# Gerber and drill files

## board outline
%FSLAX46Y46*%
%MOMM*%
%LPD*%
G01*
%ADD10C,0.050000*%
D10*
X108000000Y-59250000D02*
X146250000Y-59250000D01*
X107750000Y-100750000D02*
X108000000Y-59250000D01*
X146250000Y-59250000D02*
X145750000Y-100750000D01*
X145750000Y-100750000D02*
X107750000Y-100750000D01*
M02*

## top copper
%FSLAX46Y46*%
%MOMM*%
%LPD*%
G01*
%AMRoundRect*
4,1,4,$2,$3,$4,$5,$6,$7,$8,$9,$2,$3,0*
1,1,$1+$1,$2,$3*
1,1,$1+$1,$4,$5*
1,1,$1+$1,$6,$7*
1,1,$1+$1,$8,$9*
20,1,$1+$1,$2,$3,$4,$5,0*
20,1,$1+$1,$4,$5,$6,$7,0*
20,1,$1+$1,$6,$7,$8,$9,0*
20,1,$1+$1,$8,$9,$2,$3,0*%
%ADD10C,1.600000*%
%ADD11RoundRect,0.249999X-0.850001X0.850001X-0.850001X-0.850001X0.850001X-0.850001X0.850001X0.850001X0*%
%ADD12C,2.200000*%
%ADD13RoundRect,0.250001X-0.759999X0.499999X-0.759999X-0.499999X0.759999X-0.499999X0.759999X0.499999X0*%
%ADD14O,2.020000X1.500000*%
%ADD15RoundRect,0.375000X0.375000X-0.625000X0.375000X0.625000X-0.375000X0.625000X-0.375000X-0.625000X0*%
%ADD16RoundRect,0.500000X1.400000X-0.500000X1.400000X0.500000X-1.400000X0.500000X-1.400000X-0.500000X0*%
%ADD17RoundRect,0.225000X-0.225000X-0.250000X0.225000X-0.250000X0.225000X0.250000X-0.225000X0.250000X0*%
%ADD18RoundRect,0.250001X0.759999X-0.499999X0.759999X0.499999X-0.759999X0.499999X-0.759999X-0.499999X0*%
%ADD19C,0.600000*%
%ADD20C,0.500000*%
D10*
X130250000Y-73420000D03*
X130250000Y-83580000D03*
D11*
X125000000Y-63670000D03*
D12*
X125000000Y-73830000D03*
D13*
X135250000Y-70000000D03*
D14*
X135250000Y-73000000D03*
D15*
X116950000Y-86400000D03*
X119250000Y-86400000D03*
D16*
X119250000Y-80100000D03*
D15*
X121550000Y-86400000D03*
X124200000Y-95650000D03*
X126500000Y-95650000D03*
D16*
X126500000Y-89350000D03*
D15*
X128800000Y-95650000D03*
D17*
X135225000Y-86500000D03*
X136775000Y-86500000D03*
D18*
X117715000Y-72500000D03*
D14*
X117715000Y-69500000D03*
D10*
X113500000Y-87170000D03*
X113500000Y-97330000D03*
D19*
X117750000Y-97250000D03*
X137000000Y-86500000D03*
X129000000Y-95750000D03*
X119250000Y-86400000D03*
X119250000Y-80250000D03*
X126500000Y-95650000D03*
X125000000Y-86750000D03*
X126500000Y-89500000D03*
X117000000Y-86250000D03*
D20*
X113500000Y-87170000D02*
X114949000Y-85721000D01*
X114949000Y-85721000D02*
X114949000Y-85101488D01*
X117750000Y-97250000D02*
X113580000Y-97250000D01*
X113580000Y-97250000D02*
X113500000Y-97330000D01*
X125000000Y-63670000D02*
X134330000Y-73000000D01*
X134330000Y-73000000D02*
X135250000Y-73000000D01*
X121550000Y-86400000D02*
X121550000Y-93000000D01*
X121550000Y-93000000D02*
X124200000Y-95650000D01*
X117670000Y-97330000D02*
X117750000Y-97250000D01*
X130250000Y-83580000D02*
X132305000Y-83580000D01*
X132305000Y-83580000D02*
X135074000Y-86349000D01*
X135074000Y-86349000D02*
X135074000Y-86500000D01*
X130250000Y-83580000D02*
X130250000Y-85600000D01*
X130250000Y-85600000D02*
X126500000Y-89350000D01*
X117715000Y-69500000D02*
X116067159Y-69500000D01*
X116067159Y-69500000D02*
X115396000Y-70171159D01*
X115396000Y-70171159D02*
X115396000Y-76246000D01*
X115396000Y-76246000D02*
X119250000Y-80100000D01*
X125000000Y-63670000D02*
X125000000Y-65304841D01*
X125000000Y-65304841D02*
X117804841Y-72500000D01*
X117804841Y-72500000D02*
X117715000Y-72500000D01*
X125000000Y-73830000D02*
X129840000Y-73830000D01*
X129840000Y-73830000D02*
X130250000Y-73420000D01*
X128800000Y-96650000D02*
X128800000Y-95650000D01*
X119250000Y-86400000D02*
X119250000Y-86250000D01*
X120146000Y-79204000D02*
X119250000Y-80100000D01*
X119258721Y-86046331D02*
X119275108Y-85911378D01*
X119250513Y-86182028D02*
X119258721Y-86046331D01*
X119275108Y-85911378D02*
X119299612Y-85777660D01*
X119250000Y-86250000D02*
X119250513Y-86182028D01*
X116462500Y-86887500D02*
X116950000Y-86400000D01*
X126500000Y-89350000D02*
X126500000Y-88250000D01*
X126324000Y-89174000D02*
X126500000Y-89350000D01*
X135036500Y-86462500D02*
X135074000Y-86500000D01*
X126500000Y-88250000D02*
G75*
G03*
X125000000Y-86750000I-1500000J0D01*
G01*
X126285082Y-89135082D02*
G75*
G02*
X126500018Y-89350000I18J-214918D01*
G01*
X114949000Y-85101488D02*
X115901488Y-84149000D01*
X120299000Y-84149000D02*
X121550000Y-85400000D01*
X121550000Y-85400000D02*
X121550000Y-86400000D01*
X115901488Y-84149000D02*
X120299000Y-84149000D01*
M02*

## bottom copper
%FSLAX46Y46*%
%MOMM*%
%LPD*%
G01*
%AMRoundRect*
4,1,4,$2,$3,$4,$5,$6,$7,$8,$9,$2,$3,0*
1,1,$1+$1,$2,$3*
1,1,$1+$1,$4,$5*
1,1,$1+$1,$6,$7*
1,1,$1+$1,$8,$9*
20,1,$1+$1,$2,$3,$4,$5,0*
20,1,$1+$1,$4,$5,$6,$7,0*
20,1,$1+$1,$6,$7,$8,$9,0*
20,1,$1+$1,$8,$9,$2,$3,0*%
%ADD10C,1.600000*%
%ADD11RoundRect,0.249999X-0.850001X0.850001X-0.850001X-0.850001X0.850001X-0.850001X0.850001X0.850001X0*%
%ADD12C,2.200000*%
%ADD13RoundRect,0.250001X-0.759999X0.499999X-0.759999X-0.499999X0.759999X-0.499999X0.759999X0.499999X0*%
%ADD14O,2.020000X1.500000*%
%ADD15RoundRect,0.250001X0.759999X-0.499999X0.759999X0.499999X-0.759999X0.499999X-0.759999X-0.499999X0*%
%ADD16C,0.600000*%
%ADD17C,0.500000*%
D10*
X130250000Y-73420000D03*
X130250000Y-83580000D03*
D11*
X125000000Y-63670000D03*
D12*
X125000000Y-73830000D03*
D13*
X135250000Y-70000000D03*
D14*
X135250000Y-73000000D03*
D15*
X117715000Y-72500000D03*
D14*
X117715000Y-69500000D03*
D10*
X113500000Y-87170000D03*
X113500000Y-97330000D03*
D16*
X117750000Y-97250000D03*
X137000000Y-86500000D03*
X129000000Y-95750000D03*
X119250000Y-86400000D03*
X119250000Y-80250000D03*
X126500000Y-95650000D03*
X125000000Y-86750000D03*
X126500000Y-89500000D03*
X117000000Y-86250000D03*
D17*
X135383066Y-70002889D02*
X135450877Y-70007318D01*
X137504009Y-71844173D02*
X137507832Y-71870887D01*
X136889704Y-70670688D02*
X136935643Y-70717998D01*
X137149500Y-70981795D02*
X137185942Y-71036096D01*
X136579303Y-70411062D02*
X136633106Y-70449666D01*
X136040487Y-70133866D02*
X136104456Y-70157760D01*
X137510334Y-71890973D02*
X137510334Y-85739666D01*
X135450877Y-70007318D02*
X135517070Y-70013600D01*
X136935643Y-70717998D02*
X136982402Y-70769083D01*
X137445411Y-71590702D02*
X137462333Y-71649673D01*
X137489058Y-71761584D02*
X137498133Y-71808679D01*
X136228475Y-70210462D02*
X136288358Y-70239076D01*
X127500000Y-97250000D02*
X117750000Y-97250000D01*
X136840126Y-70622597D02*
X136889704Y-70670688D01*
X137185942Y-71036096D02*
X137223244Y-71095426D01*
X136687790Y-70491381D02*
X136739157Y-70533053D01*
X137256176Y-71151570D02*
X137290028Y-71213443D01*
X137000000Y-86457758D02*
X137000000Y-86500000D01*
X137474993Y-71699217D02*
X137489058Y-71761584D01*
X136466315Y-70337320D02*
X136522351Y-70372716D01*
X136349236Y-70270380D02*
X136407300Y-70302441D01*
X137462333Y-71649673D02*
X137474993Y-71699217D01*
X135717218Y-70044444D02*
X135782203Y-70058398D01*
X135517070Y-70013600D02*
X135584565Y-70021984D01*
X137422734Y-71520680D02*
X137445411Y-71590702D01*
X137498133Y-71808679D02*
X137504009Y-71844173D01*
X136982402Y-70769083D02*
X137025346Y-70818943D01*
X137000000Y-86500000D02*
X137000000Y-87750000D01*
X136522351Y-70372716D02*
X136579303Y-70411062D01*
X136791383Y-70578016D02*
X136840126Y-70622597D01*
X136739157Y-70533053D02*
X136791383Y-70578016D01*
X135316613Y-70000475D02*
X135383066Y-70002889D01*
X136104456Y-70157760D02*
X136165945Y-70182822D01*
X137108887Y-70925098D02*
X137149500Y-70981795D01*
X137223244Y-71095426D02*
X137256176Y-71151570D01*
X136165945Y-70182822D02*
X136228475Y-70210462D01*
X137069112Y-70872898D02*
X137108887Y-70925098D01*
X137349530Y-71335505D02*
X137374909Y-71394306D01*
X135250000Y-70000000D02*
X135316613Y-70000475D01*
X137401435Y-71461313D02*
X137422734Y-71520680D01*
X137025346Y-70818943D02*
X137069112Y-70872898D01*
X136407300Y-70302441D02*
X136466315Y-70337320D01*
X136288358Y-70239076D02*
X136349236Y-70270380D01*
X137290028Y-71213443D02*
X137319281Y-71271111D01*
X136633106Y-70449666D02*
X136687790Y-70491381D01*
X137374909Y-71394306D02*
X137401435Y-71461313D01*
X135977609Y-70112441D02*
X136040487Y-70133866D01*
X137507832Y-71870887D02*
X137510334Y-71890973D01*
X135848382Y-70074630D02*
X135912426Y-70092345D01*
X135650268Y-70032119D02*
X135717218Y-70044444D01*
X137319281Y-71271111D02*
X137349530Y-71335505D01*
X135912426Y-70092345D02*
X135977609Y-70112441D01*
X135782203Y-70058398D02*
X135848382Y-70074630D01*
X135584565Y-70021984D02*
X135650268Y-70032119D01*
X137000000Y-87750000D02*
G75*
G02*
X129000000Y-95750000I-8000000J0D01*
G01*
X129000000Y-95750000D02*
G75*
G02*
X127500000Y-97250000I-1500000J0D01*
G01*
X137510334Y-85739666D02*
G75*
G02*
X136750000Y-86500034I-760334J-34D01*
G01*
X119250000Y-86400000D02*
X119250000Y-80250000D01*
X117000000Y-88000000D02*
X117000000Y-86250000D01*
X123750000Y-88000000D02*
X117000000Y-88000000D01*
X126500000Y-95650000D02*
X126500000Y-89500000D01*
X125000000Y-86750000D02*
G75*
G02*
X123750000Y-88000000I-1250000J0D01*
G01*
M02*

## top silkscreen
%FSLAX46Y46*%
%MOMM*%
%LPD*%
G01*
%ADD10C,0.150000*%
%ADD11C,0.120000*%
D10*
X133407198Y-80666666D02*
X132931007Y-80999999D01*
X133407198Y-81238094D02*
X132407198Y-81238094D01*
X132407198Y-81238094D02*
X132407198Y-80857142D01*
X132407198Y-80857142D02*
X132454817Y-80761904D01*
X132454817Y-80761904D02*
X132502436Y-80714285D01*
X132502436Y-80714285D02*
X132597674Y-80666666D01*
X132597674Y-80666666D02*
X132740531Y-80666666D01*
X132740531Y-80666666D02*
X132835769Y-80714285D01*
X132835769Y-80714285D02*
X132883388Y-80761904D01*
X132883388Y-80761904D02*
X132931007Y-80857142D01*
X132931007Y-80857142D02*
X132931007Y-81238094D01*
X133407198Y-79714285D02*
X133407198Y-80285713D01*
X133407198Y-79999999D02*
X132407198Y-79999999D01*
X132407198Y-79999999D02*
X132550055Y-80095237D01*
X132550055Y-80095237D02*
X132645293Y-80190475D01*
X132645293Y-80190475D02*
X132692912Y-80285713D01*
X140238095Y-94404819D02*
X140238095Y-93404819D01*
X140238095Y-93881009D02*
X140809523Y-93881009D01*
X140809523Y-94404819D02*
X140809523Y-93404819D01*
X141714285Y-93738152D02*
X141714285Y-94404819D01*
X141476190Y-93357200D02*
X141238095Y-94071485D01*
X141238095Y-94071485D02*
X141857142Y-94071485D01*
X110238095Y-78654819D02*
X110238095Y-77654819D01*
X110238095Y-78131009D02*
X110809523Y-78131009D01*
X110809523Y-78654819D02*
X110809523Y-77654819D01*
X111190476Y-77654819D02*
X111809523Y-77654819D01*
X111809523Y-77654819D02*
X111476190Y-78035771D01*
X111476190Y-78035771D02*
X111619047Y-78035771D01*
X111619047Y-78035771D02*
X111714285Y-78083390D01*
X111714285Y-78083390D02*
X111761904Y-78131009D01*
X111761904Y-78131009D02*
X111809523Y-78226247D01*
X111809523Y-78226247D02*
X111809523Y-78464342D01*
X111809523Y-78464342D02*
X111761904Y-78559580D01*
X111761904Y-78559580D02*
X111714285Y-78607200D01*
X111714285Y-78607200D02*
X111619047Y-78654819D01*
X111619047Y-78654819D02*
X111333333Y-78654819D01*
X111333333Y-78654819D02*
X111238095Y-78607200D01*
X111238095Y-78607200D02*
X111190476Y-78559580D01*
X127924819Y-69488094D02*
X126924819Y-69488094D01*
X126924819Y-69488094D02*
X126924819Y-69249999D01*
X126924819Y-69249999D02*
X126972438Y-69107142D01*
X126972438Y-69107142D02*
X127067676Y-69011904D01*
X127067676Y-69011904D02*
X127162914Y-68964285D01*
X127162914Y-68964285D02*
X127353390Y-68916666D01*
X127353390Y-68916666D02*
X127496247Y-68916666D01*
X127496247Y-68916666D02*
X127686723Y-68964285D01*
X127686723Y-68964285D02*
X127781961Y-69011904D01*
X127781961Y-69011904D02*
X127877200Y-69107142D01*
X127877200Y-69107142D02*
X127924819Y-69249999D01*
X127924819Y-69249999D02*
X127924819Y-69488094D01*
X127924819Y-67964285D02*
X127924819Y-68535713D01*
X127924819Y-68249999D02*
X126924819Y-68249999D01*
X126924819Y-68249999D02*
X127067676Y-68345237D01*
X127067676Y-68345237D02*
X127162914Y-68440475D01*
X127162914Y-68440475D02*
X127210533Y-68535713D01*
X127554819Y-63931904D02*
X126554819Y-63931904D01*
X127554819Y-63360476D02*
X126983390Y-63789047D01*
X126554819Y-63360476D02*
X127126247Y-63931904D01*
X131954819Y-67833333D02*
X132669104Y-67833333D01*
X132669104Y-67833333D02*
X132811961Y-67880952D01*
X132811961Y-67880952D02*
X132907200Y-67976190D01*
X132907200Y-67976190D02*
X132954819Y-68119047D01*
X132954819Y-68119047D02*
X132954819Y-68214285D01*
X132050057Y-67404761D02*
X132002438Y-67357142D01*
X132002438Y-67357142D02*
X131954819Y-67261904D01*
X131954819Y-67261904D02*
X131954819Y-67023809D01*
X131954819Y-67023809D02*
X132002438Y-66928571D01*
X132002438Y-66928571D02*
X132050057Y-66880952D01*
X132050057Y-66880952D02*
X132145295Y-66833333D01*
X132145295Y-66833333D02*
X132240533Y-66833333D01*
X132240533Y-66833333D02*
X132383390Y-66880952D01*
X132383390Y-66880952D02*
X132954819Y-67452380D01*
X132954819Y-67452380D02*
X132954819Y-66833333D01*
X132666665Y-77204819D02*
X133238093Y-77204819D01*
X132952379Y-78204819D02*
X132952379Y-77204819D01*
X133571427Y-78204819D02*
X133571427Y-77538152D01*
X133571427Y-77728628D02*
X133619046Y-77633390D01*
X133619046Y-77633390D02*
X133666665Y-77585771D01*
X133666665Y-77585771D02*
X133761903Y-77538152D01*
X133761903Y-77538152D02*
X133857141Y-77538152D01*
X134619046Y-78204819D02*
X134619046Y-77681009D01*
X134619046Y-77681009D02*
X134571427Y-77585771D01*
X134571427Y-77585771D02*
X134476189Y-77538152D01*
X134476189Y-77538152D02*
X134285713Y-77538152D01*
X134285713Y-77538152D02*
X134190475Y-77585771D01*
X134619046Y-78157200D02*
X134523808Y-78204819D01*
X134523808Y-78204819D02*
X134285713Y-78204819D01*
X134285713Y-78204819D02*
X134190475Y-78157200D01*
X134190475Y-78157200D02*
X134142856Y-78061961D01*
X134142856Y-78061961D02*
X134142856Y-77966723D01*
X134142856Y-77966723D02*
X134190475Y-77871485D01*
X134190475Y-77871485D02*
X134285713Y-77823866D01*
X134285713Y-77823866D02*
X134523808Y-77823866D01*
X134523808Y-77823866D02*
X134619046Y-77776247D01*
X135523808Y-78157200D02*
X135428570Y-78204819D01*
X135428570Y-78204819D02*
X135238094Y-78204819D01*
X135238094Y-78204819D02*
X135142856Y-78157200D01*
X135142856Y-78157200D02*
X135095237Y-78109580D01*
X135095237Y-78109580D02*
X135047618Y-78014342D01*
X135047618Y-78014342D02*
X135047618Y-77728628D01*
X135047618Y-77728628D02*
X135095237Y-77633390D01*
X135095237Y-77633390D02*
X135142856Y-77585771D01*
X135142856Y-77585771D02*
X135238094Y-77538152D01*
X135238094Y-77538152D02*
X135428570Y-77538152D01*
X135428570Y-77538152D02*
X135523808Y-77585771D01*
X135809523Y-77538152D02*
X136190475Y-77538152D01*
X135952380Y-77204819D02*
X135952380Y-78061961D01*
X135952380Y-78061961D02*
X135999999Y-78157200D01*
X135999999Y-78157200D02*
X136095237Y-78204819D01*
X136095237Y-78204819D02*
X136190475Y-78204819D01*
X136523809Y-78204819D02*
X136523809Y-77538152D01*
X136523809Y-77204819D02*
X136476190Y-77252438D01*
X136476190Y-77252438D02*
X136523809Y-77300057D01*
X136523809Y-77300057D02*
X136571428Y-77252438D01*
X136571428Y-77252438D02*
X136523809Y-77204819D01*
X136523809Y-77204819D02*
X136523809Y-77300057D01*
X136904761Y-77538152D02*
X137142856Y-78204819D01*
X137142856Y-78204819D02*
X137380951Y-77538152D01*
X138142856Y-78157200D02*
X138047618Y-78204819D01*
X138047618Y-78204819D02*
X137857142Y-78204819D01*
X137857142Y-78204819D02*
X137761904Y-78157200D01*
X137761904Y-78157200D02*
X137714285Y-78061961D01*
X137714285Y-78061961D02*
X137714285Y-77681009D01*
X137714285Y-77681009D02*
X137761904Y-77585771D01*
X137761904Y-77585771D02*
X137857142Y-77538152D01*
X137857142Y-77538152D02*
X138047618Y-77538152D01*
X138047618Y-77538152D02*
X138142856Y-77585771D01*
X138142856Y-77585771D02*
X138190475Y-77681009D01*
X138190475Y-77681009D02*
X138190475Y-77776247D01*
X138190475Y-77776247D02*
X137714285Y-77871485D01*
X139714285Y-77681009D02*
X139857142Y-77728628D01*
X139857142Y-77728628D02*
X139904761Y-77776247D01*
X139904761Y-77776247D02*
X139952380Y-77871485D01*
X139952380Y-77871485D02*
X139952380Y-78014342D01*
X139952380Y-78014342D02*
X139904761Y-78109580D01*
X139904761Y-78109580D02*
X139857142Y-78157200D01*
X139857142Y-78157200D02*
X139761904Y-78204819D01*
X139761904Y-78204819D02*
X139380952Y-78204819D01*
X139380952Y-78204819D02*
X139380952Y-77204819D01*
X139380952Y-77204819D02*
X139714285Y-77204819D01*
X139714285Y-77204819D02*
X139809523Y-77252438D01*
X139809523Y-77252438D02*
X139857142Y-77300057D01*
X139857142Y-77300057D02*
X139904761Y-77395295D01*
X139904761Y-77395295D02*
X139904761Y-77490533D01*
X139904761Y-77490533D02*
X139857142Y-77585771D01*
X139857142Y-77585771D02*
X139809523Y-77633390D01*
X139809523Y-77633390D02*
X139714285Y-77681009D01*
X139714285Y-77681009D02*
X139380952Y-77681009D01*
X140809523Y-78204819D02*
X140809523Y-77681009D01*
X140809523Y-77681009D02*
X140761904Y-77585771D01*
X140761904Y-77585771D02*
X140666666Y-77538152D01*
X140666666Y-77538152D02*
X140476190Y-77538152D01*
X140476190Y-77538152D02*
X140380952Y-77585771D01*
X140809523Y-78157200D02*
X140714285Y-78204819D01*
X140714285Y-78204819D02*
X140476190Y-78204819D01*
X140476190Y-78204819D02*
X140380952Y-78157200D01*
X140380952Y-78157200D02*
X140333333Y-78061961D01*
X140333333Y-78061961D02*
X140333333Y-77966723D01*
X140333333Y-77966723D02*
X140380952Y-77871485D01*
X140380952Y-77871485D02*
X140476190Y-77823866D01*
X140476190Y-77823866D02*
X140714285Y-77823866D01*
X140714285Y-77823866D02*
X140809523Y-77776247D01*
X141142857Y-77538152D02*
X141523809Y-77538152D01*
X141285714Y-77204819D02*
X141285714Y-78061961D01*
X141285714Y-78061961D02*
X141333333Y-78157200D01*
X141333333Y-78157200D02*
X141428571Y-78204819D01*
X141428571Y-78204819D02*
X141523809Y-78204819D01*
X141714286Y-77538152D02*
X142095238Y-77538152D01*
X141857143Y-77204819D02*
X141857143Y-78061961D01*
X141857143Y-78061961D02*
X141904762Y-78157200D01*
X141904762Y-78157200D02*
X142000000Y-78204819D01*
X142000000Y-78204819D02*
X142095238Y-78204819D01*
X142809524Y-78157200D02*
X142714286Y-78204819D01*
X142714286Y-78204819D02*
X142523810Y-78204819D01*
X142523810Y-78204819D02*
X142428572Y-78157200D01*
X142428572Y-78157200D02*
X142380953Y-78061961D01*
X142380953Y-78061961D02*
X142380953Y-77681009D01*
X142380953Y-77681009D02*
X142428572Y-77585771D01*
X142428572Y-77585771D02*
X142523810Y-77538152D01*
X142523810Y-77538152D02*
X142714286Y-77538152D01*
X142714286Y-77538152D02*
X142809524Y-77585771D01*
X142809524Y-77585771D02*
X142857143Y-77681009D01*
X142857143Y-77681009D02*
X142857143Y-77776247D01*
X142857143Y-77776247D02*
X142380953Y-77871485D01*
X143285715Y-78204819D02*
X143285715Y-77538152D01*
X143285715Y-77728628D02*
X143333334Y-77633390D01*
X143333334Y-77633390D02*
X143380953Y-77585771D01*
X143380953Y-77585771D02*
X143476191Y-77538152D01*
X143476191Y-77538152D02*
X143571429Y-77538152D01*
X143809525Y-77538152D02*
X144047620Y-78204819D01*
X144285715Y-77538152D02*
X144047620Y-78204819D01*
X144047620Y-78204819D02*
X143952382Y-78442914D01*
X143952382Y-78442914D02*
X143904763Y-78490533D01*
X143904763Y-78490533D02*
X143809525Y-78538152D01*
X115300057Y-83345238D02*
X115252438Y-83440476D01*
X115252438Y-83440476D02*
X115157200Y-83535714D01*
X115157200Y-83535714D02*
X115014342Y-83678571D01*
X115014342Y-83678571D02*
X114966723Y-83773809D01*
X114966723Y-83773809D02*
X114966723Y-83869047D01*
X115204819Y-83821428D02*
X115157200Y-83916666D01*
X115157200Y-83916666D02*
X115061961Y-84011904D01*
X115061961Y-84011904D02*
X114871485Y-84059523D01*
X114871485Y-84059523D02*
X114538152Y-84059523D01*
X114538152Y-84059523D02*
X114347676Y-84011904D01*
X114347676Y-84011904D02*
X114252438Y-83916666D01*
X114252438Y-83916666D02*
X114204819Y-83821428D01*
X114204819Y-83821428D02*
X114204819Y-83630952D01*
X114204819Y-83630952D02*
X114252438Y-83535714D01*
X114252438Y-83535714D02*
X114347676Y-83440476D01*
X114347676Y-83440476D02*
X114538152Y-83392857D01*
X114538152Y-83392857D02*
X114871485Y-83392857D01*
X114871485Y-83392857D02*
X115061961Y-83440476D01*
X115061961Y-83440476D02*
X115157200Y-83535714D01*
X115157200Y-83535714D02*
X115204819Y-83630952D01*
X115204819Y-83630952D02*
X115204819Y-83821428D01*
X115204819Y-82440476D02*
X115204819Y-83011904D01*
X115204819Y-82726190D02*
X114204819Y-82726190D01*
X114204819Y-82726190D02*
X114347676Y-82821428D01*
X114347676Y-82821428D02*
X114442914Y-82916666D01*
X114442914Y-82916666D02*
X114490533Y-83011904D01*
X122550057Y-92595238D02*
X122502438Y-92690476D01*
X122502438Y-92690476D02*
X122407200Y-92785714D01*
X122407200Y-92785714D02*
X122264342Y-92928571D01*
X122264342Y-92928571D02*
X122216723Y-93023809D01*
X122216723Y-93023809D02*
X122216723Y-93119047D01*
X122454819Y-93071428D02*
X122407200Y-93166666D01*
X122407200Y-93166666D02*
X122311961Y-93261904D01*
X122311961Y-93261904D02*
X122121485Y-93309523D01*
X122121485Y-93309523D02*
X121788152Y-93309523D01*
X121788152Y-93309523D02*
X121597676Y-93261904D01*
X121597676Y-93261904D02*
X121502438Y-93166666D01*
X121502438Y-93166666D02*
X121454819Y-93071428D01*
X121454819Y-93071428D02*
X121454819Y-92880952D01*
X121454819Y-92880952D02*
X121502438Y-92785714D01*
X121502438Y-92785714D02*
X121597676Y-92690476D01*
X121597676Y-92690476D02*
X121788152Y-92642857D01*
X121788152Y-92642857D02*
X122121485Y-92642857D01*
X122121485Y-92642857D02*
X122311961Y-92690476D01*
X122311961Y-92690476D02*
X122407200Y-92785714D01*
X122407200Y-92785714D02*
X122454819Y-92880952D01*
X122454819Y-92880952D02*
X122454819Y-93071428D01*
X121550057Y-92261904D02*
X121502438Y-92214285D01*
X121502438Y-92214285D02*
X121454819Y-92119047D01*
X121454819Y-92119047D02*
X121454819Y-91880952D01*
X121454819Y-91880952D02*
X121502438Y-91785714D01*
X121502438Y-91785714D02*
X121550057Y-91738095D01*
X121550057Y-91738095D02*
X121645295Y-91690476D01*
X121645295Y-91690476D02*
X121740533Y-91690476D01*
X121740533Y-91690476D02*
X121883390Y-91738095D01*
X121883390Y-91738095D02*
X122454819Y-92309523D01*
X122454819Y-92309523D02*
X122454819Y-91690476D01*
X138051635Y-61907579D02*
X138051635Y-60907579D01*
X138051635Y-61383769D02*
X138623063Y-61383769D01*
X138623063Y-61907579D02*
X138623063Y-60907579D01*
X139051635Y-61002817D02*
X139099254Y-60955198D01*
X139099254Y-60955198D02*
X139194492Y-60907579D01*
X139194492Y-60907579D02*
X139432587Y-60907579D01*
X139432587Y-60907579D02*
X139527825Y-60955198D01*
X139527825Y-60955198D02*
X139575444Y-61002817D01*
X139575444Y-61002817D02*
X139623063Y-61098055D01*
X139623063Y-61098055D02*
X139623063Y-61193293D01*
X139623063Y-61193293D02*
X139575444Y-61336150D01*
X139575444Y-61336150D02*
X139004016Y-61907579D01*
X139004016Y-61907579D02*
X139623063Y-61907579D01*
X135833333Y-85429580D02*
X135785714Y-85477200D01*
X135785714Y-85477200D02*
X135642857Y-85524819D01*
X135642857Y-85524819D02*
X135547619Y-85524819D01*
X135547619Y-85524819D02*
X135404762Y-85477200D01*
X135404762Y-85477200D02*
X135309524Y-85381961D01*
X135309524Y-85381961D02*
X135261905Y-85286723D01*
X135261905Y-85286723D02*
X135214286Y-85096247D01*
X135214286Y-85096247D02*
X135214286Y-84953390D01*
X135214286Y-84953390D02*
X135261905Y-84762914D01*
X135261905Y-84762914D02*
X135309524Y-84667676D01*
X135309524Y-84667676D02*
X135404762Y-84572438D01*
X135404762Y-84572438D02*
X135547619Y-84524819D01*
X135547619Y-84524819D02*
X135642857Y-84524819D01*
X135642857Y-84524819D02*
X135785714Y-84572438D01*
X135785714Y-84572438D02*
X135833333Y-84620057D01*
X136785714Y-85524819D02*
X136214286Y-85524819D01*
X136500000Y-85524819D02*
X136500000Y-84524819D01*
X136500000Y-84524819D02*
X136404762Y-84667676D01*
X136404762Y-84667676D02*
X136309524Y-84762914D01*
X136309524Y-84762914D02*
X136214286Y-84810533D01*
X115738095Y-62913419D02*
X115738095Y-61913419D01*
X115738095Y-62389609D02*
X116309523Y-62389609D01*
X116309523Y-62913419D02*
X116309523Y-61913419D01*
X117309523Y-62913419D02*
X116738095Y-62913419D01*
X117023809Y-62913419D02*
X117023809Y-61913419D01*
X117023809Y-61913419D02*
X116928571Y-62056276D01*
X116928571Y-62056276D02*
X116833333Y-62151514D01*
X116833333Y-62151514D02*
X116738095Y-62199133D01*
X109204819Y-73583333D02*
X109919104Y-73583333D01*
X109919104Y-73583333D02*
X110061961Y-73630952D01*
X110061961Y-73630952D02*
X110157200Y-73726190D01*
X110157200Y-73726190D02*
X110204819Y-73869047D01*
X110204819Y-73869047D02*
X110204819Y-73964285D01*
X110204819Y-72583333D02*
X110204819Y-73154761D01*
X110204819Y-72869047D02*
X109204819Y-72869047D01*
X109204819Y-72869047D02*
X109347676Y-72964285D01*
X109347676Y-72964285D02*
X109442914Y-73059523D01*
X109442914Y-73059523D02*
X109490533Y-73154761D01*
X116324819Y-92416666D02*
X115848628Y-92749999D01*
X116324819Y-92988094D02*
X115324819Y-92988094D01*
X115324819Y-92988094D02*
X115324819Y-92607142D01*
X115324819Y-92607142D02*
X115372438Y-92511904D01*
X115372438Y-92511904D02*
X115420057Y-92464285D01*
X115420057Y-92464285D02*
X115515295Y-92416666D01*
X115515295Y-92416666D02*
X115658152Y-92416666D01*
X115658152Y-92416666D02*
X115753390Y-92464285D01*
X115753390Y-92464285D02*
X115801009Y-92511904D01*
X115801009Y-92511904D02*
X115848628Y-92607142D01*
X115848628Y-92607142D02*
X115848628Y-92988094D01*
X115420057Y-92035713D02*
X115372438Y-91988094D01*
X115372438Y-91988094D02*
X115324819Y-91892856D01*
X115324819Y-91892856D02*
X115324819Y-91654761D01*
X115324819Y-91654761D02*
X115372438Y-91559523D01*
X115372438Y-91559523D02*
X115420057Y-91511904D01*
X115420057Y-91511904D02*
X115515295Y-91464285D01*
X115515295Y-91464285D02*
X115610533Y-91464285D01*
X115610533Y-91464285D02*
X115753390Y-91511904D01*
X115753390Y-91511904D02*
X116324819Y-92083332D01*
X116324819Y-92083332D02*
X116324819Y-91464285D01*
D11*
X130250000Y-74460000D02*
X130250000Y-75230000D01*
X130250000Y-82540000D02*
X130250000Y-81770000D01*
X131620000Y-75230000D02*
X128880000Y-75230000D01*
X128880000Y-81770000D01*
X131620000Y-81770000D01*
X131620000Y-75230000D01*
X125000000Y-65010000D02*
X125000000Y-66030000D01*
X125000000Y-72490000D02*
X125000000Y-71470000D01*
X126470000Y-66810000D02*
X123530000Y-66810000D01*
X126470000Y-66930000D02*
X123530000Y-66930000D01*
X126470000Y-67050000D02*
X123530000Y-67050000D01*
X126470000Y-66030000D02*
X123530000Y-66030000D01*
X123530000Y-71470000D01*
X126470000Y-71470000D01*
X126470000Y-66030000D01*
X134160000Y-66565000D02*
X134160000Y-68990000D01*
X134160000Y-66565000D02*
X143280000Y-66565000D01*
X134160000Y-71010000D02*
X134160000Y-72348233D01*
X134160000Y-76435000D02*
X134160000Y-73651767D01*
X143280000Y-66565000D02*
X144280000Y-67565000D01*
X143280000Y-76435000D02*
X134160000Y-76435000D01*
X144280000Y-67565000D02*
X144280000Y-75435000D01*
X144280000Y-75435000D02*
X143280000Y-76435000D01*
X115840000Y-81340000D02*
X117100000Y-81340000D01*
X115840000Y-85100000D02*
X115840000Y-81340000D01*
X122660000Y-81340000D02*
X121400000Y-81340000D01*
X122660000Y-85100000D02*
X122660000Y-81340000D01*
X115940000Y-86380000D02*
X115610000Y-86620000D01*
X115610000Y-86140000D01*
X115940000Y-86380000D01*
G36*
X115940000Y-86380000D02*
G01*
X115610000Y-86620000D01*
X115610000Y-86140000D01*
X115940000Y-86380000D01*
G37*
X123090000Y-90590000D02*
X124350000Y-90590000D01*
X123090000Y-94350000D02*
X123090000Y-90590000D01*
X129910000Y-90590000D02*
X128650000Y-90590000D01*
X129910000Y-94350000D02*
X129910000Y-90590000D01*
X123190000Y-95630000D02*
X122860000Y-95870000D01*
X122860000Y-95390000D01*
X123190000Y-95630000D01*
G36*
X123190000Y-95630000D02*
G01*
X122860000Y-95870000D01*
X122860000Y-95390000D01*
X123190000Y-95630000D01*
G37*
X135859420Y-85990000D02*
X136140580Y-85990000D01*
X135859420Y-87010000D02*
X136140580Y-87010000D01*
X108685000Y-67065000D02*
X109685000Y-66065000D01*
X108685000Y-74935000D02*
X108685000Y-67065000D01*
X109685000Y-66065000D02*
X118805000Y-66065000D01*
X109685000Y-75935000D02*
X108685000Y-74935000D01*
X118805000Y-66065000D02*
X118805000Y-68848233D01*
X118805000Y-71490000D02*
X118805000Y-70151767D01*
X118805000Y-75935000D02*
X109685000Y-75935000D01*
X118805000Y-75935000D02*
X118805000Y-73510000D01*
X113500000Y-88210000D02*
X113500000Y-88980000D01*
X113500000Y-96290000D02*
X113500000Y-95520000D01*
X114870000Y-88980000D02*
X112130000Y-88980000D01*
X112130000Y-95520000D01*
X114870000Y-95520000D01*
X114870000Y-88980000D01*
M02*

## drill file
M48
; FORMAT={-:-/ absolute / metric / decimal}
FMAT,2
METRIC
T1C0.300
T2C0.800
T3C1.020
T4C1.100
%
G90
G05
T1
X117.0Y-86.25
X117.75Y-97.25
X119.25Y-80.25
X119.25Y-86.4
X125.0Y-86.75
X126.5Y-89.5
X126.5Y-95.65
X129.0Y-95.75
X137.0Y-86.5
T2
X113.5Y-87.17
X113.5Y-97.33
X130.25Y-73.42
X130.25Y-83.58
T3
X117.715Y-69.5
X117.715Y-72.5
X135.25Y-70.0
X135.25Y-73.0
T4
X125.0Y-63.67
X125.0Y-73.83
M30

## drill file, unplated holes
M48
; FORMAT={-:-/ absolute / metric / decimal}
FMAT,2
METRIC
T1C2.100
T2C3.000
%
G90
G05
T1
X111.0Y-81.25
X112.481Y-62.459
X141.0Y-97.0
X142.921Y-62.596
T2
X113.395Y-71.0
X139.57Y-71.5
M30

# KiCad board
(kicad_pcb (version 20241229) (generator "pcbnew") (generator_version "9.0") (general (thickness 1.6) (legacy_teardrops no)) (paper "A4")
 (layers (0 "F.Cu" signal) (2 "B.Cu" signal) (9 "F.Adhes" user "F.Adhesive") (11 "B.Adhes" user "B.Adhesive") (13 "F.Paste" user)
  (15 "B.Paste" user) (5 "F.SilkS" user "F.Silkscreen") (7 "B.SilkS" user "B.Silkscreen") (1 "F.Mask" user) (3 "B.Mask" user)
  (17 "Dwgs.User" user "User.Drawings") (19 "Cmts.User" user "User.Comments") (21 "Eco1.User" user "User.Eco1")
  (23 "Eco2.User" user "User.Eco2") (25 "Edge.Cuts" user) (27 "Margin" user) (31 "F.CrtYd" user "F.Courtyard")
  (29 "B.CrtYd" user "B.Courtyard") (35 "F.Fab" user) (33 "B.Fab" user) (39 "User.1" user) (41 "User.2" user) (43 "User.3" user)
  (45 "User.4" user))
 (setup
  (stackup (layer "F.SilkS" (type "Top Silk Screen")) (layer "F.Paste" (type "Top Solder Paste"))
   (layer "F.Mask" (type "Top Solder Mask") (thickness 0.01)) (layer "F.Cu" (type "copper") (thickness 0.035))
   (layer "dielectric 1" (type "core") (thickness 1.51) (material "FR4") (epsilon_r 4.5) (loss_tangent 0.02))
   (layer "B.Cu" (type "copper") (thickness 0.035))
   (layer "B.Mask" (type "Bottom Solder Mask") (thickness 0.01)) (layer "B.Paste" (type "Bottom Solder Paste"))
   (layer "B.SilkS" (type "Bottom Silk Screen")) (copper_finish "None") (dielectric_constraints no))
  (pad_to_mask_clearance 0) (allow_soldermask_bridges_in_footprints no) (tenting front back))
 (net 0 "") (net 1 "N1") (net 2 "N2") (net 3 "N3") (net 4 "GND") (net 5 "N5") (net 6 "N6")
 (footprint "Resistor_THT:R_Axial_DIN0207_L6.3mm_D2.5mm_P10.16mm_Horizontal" (layer "F.Cu") (at 130.25 73.42 -90)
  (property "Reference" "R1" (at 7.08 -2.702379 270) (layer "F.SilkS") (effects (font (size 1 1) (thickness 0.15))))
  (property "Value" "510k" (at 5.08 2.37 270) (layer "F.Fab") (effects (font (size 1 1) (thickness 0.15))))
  (fp_line (start 1.04 0) (end 1.81 0) (stroke (width 0.12) (type solid)) (layer "F.SilkS"))
  (fp_line (start 9.12 0) (end 8.35 0) (stroke (width 0.12) (type solid)) (layer "F.SilkS"))
  (fp_rect (start 1.81 -1.37) (end 8.35 1.37) (stroke (width 0.12) (type solid)) (fill no) (layer "F.SilkS"))
  (pad "1" thru_hole circle (at 0 0 270) (size 1.6 1.6) (drill 0.8) (layers "*.Cu" "*.Mask") (remove_unused_layers no) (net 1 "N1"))
  (pad "2" thru_hole circle (at 10.16 0 270) (size 1.6 1.6) (drill 0.8) (layers "*.Cu" "*.Mask") (remove_unused_layers no) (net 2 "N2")))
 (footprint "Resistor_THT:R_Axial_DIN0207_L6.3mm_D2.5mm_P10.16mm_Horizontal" (layer "F.Cu") (at 113.5 87.17 -90)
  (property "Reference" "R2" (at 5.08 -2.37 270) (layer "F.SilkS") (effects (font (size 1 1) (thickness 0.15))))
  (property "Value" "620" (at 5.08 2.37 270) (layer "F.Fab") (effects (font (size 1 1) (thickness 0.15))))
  (fp_line (start 1.04 0) (end 1.81 0) (stroke (width 0.12) (type solid)) (layer "F.SilkS"))
  (fp_line (start 9.12 0) (end 8.35 0) (stroke (width 0.12) (type solid)) (layer "F.SilkS"))
  (fp_rect (start 1.81 -1.37) (end 8.35 1.37) (stroke (width 0.12) (type solid)) (fill no) (layer "F.SilkS"))
  (pad "1" thru_hole circle (at 0 0 270) (size 1.6 1.6) (drill 0.8) (layers "*.Cu" "*.Mask") (remove_unused_layers no) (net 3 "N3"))
  (pad "2" thru_hole circle (at 10.16 0 270) (size 1.6 1.6) (drill 0.8) (layers "*.Cu" "*.Mask") (remove_unused_layers no) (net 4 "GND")))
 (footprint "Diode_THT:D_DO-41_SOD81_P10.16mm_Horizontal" (layer "F.Cu") (at 125 63.67 -90)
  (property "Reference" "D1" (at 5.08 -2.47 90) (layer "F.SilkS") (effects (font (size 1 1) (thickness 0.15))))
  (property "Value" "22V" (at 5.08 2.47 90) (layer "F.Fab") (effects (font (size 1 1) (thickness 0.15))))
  (fp_line (start 1.34 0) (end 2.36 0) (stroke (width 0.12) (type solid)) (layer "F.SilkS"))
  (fp_line (start 8.82 0) (end 7.8 0) (stroke (width 0.12) (type solid)) (layer "F.SilkS"))
  (fp_line (start 3.14 -1.47) (end 3.14 1.47) (stroke (width 0.12) (type solid)) (layer "F.SilkS"))
  (fp_line (start 3.26 -1.47) (end 3.26 1.47) (stroke (width 0.12) (type solid)) (layer "F.SilkS"))
  (fp_line (start 3.38 -1.47) (end 3.38 1.47) (stroke (width 0.12) (type solid)) (layer "F.SilkS"))
  (fp_rect (start 2.36 -1.47) (end 7.8 1.47) (stroke (width 0.12) (type solid)) (fill no) (layer "F.SilkS"))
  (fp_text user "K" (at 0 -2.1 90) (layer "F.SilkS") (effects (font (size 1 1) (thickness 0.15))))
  (pad "1" thru_hole roundrect (at 0 0 270) (size 2.2 2.2) (drill 1.1) (layers "*.Cu" "*.Mask") (remove_unused_layers no)
   (roundrect_rratio 0.113636) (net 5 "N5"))
  (pad "2" thru_hole circle (at 10.16 0 270) (size 2.2 2.2) (drill 1.1) (layers "*.Cu" "*.Mask") (remove_unused_layers no) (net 1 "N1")))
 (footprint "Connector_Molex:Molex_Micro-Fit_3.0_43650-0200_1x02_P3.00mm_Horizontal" (layer "F.Cu") (at 135.25 70 -90)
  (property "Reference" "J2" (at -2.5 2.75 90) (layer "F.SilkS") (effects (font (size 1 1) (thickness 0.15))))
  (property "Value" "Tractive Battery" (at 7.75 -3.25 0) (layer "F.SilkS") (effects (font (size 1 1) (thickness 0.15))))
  (fp_line (start -3.435 1.09) (end -1.01 1.09) (stroke (width 0.12) (type solid)) (layer "F.SilkS"))
  (fp_line (start -3.435 1.09) (end -3.435 -8.03) (stroke (width 0.12) (type solid)) (layer "F.SilkS"))
  (fp_line (start 1.01 1.09) (end 2.348233 1.09) (stroke (width 0.12) (type solid)) (layer "F.SilkS"))
  (fp_line (start 6.435 1.09) (end 3.651767 1.09) (stroke (width 0.12) (type solid)) (layer "F.SilkS"))
  (fp_line (start -3.435 -8.03) (end -2.435 -9.03) (stroke (width 0.12) (type solid)) (layer "F.SilkS"))
  (fp_line (start 6.435 -8.03) (end 6.435 1.09) (stroke (width 0.12) (type solid)) (layer "F.SilkS"))
  (fp_line (start -2.435 -9.03) (end 5.435 -9.03) (stroke (width 0.12) (type solid)) (layer "F.SilkS"))
  (fp_line (start 5.435 -9.03) (end 6.435 -8.03) (stroke (width 0.12) (type solid)) (layer "F.SilkS"))
  (pad "" np_thru_hole circle (at 1.5 -4.32 270) (size 3 3) (drill 3) (layers "*.Cu" "*.Mask"))
  (pad "1" thru_hole roundrect (at 0 0 270) (size 1.5 2.02) (drill 1.02) (layers "*.Cu" "*.Mask") (remove_unused_layers no)
   (roundrect_rratio 0.166667) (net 4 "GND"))
  (pad "2" thru_hole oval (at 3 0 270) (size 1.5 2.02) (drill 1.02) (layers "*.Cu" "*.Mask") (remove_unused_layers no) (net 5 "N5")))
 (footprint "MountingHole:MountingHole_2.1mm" (layer "F.Cu") (at 111 81.25)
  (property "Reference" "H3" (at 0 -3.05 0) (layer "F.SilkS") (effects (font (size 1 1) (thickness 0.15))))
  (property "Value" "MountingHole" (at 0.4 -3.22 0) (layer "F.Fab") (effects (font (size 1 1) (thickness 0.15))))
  (pad "" np_thru_hole circle (at 0 0) (size 2.1 2.1) (drill 2.1) (layers "*.Cu" "*.Mask")))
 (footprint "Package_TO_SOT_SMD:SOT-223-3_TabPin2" (layer "F.Cu") (at 119.25 83.25 90)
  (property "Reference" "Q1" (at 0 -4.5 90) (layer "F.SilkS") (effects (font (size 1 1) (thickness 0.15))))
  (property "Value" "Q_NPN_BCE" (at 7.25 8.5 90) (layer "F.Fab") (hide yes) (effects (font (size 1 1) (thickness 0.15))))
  (fp_line (start 1.91 -3.41) (end 1.91 -2.15) (stroke (width 0.12) (type solid)) (layer "F.SilkS"))
  (fp_line (start -1.85 -3.41) (end 1.91 -3.41) (stroke (width 0.12) (type solid)) (layer "F.SilkS"))
  (fp_line (start 1.91 3.41) (end 1.91 2.15) (stroke (width 0.12) (type solid)) (layer "F.SilkS"))
  (fp_line (start -1.85 3.41) (end 1.91 3.41) (stroke (width 0.12) (type solid)) (layer "F.SilkS"))
  (fp_poly
   (pts (xy -3.13 -3.31) (xy -3.37 -3.64) (xy -2.89 -3.64) (xy -3.13 -3.31)) (stroke (width 0.12) (type solid)) (fill yes) (layer "F.SilkS"))
  (pad "1" smd roundrect (at -3.15 -2.3 90) (size 2 1.5) (layers "F.Cu" "F.Mask" "F.Paste") (roundrect_rratio 0.25) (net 2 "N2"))
  (pad "2" smd roundrect (at -3.15 0 90) (size 2 1.5) (layers "F.Cu" "F.Mask" "F.Paste") (roundrect_rratio 0.25) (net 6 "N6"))
  (pad "2" smd roundrect (at 3.15 0 90) (size 2 3.8) (layers "F.Cu" "F.Mask" "F.Paste") (roundrect_rratio 0.25) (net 6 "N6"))
  (pad "3" smd roundrect (at -3.15 2.3 90) (size 2 1.5) (layers "F.Cu" "F.Mask" "F.Paste") (roundrect_rratio 0.25) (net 3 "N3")))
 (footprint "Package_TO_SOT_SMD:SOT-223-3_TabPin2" (layer "F.Cu") (at 126.5 92.5 90)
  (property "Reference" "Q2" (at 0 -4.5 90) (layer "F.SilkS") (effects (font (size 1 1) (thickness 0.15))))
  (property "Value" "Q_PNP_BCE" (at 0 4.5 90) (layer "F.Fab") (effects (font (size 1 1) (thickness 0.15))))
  (fp_line (start 1.91 -3.41) (end 1.91 -2.15) (stroke (width 0.12) (type solid)) (layer "F.SilkS"))
  (fp_line (start -1.85 -3.41) (end 1.91 -3.41) (stroke (width 0.12) (type solid)) (layer "F.SilkS"))
  (fp_line (start 1.91 3.41) (end 1.91 2.15) (stroke (width 0.12) (type solid)) (layer "F.SilkS"))
  (fp_line (start -1.85 3.41) (end 1.91 3.41) (stroke (width 0.12) (type solid)) (layer "F.SilkS"))
  (fp_poly
   (pts (xy -3.13 -3.31) (xy -3.37 -3.64) (xy -2.89 -3.64) (xy -3.13 -3.31)) (stroke (width 0.12) (type solid)) (fill yes) (layer "F.SilkS"))
  (pad "1" smd roundrect (at -3.15 -2.3 90) (size 2 1.5) (layers "F.Cu" "F.Mask" "F.Paste") (roundrect_rratio 0.25) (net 3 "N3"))
  (pad "2" smd roundrect (at -3.15 0 90) (size 2 1.5) (layers "F.Cu" "F.Mask" "F.Paste") (roundrect_rratio 0.25) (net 2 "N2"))
  (pad "2" smd roundrect (at 3.15 0 90) (size 2 3.8) (layers "F.Cu" "F.Mask" "F.Paste") (roundrect_rratio 0.25) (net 2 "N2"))
  (pad "3" smd roundrect (at -3.15 2.3 90) (size 2 1.5) (layers "F.Cu" "F.Mask" "F.Paste") (roundrect_rratio 0.25) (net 4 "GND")))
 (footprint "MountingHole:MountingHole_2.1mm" (layer "F.Cu") (at 142.92072 62.59576)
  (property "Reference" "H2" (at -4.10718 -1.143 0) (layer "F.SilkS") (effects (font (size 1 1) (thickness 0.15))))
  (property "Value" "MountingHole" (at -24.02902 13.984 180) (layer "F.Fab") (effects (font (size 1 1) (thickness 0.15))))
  (pad "" np_thru_hole circle (at 0 0) (size 2.1 2.1) (drill 2.1) (layers "*.Cu" "*.Mask")))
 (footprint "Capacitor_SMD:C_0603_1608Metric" (layer "F.Cu") (at 136 86.5)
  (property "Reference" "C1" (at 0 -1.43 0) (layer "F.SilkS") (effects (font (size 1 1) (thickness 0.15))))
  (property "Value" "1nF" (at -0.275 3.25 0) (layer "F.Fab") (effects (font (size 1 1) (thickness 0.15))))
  (fp_line (start -0.14058 -0.51) (end 0.14058 -0.51) (stroke (width 0.12) (type solid)) (layer "F.SilkS"))
  (fp_line (start -0.14058 0.51) (end 0.14058 0.51) (stroke (width 0.12) (type solid)) (layer "F.SilkS"))
  (pad "1" smd roundrect (at -0.775 0) (size 0.9 0.95) (layers "F.Cu" "F.Mask" "F.Paste") (roundrect_rratio 0.25) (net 2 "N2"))
  (pad "2" smd roundrect (at 0.775 0) (size 0.9 0.95) (layers "F.Cu" "F.Mask" "F.Paste") (roundrect_rratio 0.25) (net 4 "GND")))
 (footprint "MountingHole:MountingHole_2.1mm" (layer "F.Cu") (at 112.48136 62.4586)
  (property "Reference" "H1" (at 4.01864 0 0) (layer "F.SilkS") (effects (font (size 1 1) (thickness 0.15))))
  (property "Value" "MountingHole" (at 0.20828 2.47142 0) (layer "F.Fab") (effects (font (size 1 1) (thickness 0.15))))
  (pad "" np_thru_hole circle (at 0 0) (size 2.1 2.1) (drill 2.1) (layers "*.Cu" "*.Mask")))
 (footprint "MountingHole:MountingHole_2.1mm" (layer "F.Cu") (at 141 97)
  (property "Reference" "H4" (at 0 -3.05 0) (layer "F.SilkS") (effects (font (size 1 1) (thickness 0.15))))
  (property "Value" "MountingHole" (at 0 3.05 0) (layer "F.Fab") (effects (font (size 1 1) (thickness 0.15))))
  (pad "" np_thru_hole circle (at 0 0) (size 2.1 2.1) (drill 2.1) (layers "*.Cu" "*.Mask")))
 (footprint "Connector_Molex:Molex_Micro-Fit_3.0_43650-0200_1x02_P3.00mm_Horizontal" (layer "F.Cu") (at 117.715 72.5 90)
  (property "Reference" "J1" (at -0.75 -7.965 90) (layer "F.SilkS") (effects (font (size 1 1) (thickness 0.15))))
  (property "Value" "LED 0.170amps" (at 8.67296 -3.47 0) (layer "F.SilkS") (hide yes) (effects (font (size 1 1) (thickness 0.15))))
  (fp_line (start 5.435 -9.03) (end 6.435 -8.03) (stroke (width 0.12) (type solid)) (layer "F.SilkS"))
  (fp_line (start -2.435 -9.03) (end 5.435 -9.03) (stroke (width 0.12) (type solid)) (layer "F.SilkS"))
  (fp_line (start 6.435 -8.03) (end 6.435 1.09) (stroke (width 0.12) (type solid)) (layer "F.SilkS"))
  (fp_line (start -3.435 -8.03) (end -2.435 -9.03) (stroke (width 0.12) (type solid)) (layer "F.SilkS"))
  (fp_line (start 6.435 1.09) (end 3.651767 1.09) (stroke (width 0.12) (type solid)) (layer "F.SilkS"))
  (fp_line (start 1.01 1.09) (end 2.348233 1.09) (stroke (width 0.12) (type solid)) (layer "F.SilkS"))
  (fp_line (start -3.435 1.09) (end -3.435 -8.03) (stroke (width 0.12) (type solid)) (layer "F.SilkS"))
  (fp_line (start -3.435 1.09) (end -1.01 1.09) (stroke (width 0.12) (type solid)) (layer "F.SilkS"))
  (pad "" np_thru_hole circle (at 1.5 -4.32 90) (size 3 3) (drill 3) (layers "*.Cu" "*.Mask"))
  (pad "1" thru_hole roundrect (at 0 0 90) (size 1.5 2.02) (drill 1.02) (layers "*.Cu" "*.Mask") (remove_unused_layers no)
   (roundrect_rratio 0.166667) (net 5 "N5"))
  (pad "2" thru_hole oval (at 3 0 90) (size 1.5 2.02) (drill 1.02) (layers "*.Cu" "*.Mask") (remove_unused_layers no) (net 6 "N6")))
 (gr_line (start 108 59.25) (end 146.25 59.25) (stroke (width 0.05) (type default)) (layer "Edge.Cuts"))
 (gr_line (start 107.75 100.75) (end 108 59.25) (stroke (width 0.05) (type default)) (layer "Edge.Cuts"))
 (gr_line (start 146.25 59.25) (end 145.75 100.75) (stroke (width 0.05) (type default)) (layer "Edge.Cuts"))
 (gr_line (start 145.75 100.75) (end 107.75 100.75) (stroke (width 0.05) (type default)) (layer "Edge.Cuts"))
 (segment (start 117.67 97.33) (end 117.75 97.25) (width 0.5) (layer "F.Cu") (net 4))
 (segment (start 113.58 97.25) (end 113.5 97.33) (width 0.5) (layer "F.Cu") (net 4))
 (segment (start 128.8 96.65) (end 128.8 95.65) (width 0.5) (layer "F.Cu") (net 4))
 (segment (start 117.75 97.25) (end 113.58 97.25) (width 0.5) (layer "F.Cu") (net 4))
 (via (at 117.75 97.25) (size 0.6) (drill 0.3) (layers "F.Cu" "B.Cu") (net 4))
 (via (at 137 86.5) (size 0.6) (drill 0.3) (layers "F.Cu" "B.Cu") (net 4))
 (via (at 129 95.75) (size 0.6) (drill 0.3) (layers "F.Cu" "B.Cu") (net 4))
 (segment (start 135.383066 70.002889) (end 135.450877 70.007318) (width 0.5) (layer "B.Cu") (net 4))
 (segment (start 137.504009 71.844173) (end 137.507832 71.870887) (width 0.5) (layer "B.Cu") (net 4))
 (segment (start 136.889704 70.670688) (end 136.935643 70.717998) (width 0.5) (layer "B.Cu") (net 4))
 (segment (start 137.1495 70.981795) (end 137.185942 71.036096) (width 0.5) (layer "B.Cu") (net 4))
 (segment (start 136.579303 70.411062) (end 136.633106 70.449666) (width 0.5) (layer "B.Cu") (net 4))
 (segment (start 136.040487 70.133866) (end 136.104456 70.15776) (width 0.5) (layer "B.Cu") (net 4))
 (segment (start 137.510334 71.890973) (end 137.510334 85.739666) (width 0.5) (layer "B.Cu") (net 4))
 (segment (start 135.450877 70.007318) (end 135.51707 70.0136) (width 0.5) (layer "B.Cu") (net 4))
 (segment (start 136.935643 70.717998) (end 136.982402 70.769083) (width 0.5) (layer "B.Cu") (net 4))
 (segment (start 137.445411 71.590702) (end 137.462333 71.649673) (width 0.5) (layer "B.Cu") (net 4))
 (segment (start 137.489058 71.761584) (end 137.498133 71.808679) (width 0.5) (layer "B.Cu") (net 4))
 (segment (start 136.228475 70.210462) (end 136.288358 70.239076) (width 0.5) (layer "B.Cu") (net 4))
 (segment (start 127.5 97.25) (end 117.75 97.25) (width 0.5) (layer "B.Cu") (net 4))
 (segment (start 136.840126 70.622597) (end 136.889704 70.670688) (width 0.5) (layer "B.Cu") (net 4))
 (segment (start 137.185942 71.036096) (end 137.223244 71.095426) (width 0.5) (layer "B.Cu") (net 4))
 (segment (start 136.68779 70.491381) (end 136.739157 70.533053) (width 0.5) (layer "B.Cu") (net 4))
 (segment (start 137.256176 71.15157) (end 137.290028 71.213443) (width 0.5) (layer "B.Cu") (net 4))
 (segment (start 137 86.457758) (end 137 86.5) (width 0.5) (layer "B.Cu") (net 4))
 (segment (start 137.474993 71.699217) (end 137.489058 71.761584) (width 0.5) (layer "B.Cu") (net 4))
 (segment (start 136.466315 70.33732) (end 136.522351 70.372716) (width 0.5) (layer "B.Cu") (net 4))
 (segment (start 136.349236 70.27038) (end 136.4073 70.302441) (width 0.5) (layer "B.Cu") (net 4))
 (segment (start 137.462333 71.649673) (end 137.474993 71.699217) (width 0.5) (layer "B.Cu") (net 4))
 (segment (start 135.717218 70.044444) (end 135.782203 70.058398) (width 0.5) (layer "B.Cu") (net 4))
 (segment (start 135.51707 70.0136) (end 135.584565 70.021984) (width 0.5) (layer "B.Cu") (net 4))
 (segment (start 137.422734 71.52068) (end 137.445411 71.590702) (width 0.5) (layer "B.Cu") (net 4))
 (segment (start 137.498133 71.808679) (end 137.504009 71.844173) (width 0.5) (layer "B.Cu") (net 4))
 (segment (start 136.982402 70.769083) (end 137.025346 70.818943) (width 0.5) (layer "B.Cu") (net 4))
 (segment (start 137 86.5) (end 137 87.75) (width 0.5) (layer "B.Cu") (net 4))
 (segment (start 136.522351 70.372716) (end 136.579303 70.411062) (width 0.5) (layer "B.Cu") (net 4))
 (segment (start 136.791383 70.578016) (end 136.840126 70.622597) (width 0.5) (layer "B.Cu") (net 4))
 (segment (start 136.739157 70.533053) (end 136.791383 70.578016) (width 0.5) (layer "B.Cu") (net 4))
 (segment (start 135.316613 70.000475) (end 135.383066 70.002889) (width 0.5) (layer "B.Cu") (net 4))
 (segment (start 136.104456 70.15776) (end 136.165945 70.182822) (width 0.5) (layer "B.Cu") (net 4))
 (segment (start 137.108887 70.925098) (end 137.1495 70.981795) (width 0.5) (layer "B.Cu") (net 4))
 (segment (start 137.223244 71.095426) (end 137.256176 71.15157) (width 0.5) (layer "B.Cu") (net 4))
 (segment (start 136.165945 70.182822) (end 136.228475 70.210462) (width 0.5) (layer "B.Cu") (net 4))
 (segment (start 137.069112 70.872898) (end 137.108887 70.925098) (width 0.5) (layer "B.Cu") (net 4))
 (segment (start 137.34953 71.335505) (end 137.374909 71.394306) (width 0.5) (layer "B.Cu") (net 4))
 (segment (start 135.25 70) (end 135.316613 70.000475) (width 0.5) (layer "B.Cu") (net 4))
 (segment (start 137.401435 71.461313) (end 137.422734 71.52068) (width 0.5) (layer "B.Cu") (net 4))
 (segment (start 137.025346 70.818943) (end 137.069112 70.872898) (width 0.5) (layer "B.Cu") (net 4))
 (segment (start 136.4073 70.302441) (end 136.466315 70.33732) (width 0.5) (layer "B.Cu") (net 4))
 (segment (start 136.288358 70.239076) (end 136.349236 70.27038) (width 0.5) (layer "B.Cu") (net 4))
 (segment (start 137.290028 71.213443) (end 137.319281 71.271111) (width 0.5) (layer "B.Cu") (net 4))
 (segment (start 136.633106 70.449666) (end 136.68779 70.491381) (width 0.5) (layer "B.Cu") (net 4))
 (segment (start 137.374909 71.394306) (end 137.401435 71.461313) (width 0.5) (layer "B.Cu") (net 4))
 (segment (start 135.977609 70.112441) (end 136.040487 70.133866) (width 0.5) (layer "B.Cu") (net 4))
 (segment (start 137.507832 71.870887) (end 137.510334 71.890973) (width 0.5) (layer "B.Cu") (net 4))
 (segment (start 135.848382 70.07463) (end 135.912426 70.092345) (width 0.5) (layer "B.Cu") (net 4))
 (segment (start 135.650268 70.032119) (end 135.717218 70.044444) (width 0.5) (layer "B.Cu") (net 4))
 (segment (start 137.319281 71.271111) (end 137.34953 71.335505) (width 0.5) (layer "B.Cu") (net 4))
 (segment (start 135.912426 70.092345) (end 135.977609 70.112441) (width 0.5) (layer "B.Cu") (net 4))
 (segment (start 135.782203 70.058398) (end 135.848382 70.07463) (width 0.5) (layer "B.Cu") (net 4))
 (segment (start 135.584565 70.021984) (end 135.650268 70.032119) (width 0.5) (layer "B.Cu") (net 4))
 (arc (start 137 87.75) (mid 134.656854 93.406854) (end 129 95.75) (width 0.5) (layer "B.Cu") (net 4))
 (arc (start 129 95.75) (mid 128.56066 96.81066) (end 127.5 97.25) (width 0.5) (layer "B.Cu") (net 4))
 (arc (start 137.510334 85.739666) (mid 137.287637 86.277303) (end 136.75 86.5) (width 0.5) (layer "B.Cu") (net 4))
 (segment (start 117.804841 72.5) (end 117.715 72.5) (width 0.5) (layer "F.Cu") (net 5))
 (segment (start 125 63.67) (end 125 65.304841) (width 0.5) (layer "F.Cu") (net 5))
 (segment (start 125 65.304841) (end 117.804841 72.5) (width 0.5) (layer "F.Cu") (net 5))
 (segment (start 125 63.67) (end 134.33 73) (width 0.5) (layer "F.Cu") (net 5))
 (segment (start 134.33 73) (end 135.25 73) (width 0.5) (layer "F.Cu") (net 5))
 (segment (start 129.84 73.83) (end 130.25 73.42) (width 0.5) (layer "F.Cu") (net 1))
 (segment (start 125 73.83) (end 129.84 73.83) (width 0.5) (layer "F.Cu") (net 1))
 (segment (start 119.25 86.4) (end 119.25 86.25) (width 0.5) (layer "F.Cu") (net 6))
 (segment (start 115.396 70.171159) (end 115.396 76.246) (width 0.5) (layer "F.Cu") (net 6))
 (segment (start 116.067159 69.5) (end 115.396 70.171159) (width 0.5) (layer "F.Cu") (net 6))
 (segment (start 120.146 79.204) (end 119.25 80.1) (width 0.5) (layer "F.Cu") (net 6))
 (segment (start 119.258721 86.046331) (end 119.275108 85.911378) (width 0.5) (layer "F.Cu") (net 6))
 (segment (start 119.250513 86.182028) (end 119.258721 86.046331) (width 0.5) (layer "F.Cu") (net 6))
 (segment (start 119.275108 85.911378) (end 119.299612 85.77766) (width 0.5) (layer "F.Cu") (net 6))
 (segment (start 119.25 86.25) (end 119.250513 86.182028) (width 0.5) (layer "F.Cu") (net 6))
 (segment (start 117.715 69.5) (end 116.067159 69.5) (width 0.5) (layer "F.Cu") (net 6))
 (segment (start 115.396 76.246) (end 119.25 80.1) (width 0.5) (layer "F.Cu") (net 6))
 (via (at 119.25 86.4) (size 0.6) (drill 0.3) (layers "F.Cu" "B.Cu") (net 6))
 (via (at 119.25 80.25) (size 0.6) (drill 0.3) (layers "F.Cu" "B.Cu") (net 6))
 (segment (start 119.25 86.4) (end 119.25 80.25) (width 0.5) (layer "B.Cu") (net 6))
 (segment (start 130.25 85.6) (end 126.5 89.35) (width 0.5) (layer "F.Cu") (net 2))
 (segment (start 130.25 83.58) (end 130.25 85.6) (width 0.5) (layer "F.Cu") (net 2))
 (segment (start 130.25 83.58) (end 132.305 83.58) (width 0.5) (layer "F.Cu") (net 2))
 (segment (start 116.4625 86.8875) (end 116.95 86.4) (width 0.5) (layer "F.Cu") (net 2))
 (segment (start 126.5 89.35) (end 126.5 88.25) (width 0.5) (layer "F.Cu") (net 2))
 (segment (start 126.324 89.174) (end 126.5 89.35) (width 0.5) (layer "F.Cu") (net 2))
 (segment (start 135.0365 86.4625) (end 135.074 86.5) (width 0.5) (layer "F.Cu") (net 2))
 (segment (start 132.305 83.58) (end 135.074 86.349) (width 0.5) (layer "F.Cu") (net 2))
 (segment (start 135.074 86.349) (end 135.074 86.5) (width 0.5) (layer "F.Cu") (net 2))
 (via (at 126.5 95.65) (size 0.6) (drill 0.3) (layers "F.Cu" "B.Cu") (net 2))
 (via (at 125 86.75) (size 0.6) (drill 0.3) (layers "F.Cu" "B.Cu") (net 2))
 (via (at 126.5 89.5) (size 0.6) (drill 0.3) (layers "F.Cu" "B.Cu") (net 2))
 (via (at 117 86.25) (size 0.6) (drill 0.3) (layers "F.Cu" "B.Cu") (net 2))
 (arc (start 126.5 88.25) (mid 126.06066 87.18934) (end 125 86.75) (width 0.5) (layer "F.Cu") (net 2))
 (arc (start 126.285082 89.135082) (mid 126.437052 89.19803) (end 126.5 89.35) (width 0.5) (layer "F.Cu") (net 2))
 (segment (start 117 88) (end 117 86.25) (width 0.5) (layer "B.Cu") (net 2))
 (segment (start 123.75 88) (end 117 88) (width 0.5) (layer "B.Cu") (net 2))
 (segment (start 126.5 95.65) (end 126.5 89.5) (width 0.5) (layer "B.Cu") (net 2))
 (arc (start 125 86.75) (mid 124.633883 87.633883) (end 123.75 88) (width 0.5) (layer "B.Cu") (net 2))
 (segment (start 114.949 85.101488) (end 115.901488 84.149) (width 0.5) (layer "F.Cu") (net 3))
 (segment (start 120.299 84.149) (end 121.55 85.4) (width 0.5) (layer "F.Cu") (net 3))
 (segment (start 114.949 85.721) (end 114.949 85.101488) (width 0.5) (layer "F.Cu") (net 3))
 (segment (start 121.55 85.4) (end 121.55 86.4) (width 0.5) (layer "F.Cu") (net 3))
 (segment (start 113.5 87.17) (end 114.949 85.721) (width 0.5) (layer "F.Cu") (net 3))
 (segment (start 121.55 93) (end 124.2 95.65) (width 0.5) (layer "F.Cu") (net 3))
 (segment (start 121.55 86.4) (end 121.55 93) (width 0.5) (layer "F.Cu") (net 3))
 (segment (start 115.901488 84.149) (end 120.299 84.149) (width 0.5) (layer "F.Cu") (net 3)))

